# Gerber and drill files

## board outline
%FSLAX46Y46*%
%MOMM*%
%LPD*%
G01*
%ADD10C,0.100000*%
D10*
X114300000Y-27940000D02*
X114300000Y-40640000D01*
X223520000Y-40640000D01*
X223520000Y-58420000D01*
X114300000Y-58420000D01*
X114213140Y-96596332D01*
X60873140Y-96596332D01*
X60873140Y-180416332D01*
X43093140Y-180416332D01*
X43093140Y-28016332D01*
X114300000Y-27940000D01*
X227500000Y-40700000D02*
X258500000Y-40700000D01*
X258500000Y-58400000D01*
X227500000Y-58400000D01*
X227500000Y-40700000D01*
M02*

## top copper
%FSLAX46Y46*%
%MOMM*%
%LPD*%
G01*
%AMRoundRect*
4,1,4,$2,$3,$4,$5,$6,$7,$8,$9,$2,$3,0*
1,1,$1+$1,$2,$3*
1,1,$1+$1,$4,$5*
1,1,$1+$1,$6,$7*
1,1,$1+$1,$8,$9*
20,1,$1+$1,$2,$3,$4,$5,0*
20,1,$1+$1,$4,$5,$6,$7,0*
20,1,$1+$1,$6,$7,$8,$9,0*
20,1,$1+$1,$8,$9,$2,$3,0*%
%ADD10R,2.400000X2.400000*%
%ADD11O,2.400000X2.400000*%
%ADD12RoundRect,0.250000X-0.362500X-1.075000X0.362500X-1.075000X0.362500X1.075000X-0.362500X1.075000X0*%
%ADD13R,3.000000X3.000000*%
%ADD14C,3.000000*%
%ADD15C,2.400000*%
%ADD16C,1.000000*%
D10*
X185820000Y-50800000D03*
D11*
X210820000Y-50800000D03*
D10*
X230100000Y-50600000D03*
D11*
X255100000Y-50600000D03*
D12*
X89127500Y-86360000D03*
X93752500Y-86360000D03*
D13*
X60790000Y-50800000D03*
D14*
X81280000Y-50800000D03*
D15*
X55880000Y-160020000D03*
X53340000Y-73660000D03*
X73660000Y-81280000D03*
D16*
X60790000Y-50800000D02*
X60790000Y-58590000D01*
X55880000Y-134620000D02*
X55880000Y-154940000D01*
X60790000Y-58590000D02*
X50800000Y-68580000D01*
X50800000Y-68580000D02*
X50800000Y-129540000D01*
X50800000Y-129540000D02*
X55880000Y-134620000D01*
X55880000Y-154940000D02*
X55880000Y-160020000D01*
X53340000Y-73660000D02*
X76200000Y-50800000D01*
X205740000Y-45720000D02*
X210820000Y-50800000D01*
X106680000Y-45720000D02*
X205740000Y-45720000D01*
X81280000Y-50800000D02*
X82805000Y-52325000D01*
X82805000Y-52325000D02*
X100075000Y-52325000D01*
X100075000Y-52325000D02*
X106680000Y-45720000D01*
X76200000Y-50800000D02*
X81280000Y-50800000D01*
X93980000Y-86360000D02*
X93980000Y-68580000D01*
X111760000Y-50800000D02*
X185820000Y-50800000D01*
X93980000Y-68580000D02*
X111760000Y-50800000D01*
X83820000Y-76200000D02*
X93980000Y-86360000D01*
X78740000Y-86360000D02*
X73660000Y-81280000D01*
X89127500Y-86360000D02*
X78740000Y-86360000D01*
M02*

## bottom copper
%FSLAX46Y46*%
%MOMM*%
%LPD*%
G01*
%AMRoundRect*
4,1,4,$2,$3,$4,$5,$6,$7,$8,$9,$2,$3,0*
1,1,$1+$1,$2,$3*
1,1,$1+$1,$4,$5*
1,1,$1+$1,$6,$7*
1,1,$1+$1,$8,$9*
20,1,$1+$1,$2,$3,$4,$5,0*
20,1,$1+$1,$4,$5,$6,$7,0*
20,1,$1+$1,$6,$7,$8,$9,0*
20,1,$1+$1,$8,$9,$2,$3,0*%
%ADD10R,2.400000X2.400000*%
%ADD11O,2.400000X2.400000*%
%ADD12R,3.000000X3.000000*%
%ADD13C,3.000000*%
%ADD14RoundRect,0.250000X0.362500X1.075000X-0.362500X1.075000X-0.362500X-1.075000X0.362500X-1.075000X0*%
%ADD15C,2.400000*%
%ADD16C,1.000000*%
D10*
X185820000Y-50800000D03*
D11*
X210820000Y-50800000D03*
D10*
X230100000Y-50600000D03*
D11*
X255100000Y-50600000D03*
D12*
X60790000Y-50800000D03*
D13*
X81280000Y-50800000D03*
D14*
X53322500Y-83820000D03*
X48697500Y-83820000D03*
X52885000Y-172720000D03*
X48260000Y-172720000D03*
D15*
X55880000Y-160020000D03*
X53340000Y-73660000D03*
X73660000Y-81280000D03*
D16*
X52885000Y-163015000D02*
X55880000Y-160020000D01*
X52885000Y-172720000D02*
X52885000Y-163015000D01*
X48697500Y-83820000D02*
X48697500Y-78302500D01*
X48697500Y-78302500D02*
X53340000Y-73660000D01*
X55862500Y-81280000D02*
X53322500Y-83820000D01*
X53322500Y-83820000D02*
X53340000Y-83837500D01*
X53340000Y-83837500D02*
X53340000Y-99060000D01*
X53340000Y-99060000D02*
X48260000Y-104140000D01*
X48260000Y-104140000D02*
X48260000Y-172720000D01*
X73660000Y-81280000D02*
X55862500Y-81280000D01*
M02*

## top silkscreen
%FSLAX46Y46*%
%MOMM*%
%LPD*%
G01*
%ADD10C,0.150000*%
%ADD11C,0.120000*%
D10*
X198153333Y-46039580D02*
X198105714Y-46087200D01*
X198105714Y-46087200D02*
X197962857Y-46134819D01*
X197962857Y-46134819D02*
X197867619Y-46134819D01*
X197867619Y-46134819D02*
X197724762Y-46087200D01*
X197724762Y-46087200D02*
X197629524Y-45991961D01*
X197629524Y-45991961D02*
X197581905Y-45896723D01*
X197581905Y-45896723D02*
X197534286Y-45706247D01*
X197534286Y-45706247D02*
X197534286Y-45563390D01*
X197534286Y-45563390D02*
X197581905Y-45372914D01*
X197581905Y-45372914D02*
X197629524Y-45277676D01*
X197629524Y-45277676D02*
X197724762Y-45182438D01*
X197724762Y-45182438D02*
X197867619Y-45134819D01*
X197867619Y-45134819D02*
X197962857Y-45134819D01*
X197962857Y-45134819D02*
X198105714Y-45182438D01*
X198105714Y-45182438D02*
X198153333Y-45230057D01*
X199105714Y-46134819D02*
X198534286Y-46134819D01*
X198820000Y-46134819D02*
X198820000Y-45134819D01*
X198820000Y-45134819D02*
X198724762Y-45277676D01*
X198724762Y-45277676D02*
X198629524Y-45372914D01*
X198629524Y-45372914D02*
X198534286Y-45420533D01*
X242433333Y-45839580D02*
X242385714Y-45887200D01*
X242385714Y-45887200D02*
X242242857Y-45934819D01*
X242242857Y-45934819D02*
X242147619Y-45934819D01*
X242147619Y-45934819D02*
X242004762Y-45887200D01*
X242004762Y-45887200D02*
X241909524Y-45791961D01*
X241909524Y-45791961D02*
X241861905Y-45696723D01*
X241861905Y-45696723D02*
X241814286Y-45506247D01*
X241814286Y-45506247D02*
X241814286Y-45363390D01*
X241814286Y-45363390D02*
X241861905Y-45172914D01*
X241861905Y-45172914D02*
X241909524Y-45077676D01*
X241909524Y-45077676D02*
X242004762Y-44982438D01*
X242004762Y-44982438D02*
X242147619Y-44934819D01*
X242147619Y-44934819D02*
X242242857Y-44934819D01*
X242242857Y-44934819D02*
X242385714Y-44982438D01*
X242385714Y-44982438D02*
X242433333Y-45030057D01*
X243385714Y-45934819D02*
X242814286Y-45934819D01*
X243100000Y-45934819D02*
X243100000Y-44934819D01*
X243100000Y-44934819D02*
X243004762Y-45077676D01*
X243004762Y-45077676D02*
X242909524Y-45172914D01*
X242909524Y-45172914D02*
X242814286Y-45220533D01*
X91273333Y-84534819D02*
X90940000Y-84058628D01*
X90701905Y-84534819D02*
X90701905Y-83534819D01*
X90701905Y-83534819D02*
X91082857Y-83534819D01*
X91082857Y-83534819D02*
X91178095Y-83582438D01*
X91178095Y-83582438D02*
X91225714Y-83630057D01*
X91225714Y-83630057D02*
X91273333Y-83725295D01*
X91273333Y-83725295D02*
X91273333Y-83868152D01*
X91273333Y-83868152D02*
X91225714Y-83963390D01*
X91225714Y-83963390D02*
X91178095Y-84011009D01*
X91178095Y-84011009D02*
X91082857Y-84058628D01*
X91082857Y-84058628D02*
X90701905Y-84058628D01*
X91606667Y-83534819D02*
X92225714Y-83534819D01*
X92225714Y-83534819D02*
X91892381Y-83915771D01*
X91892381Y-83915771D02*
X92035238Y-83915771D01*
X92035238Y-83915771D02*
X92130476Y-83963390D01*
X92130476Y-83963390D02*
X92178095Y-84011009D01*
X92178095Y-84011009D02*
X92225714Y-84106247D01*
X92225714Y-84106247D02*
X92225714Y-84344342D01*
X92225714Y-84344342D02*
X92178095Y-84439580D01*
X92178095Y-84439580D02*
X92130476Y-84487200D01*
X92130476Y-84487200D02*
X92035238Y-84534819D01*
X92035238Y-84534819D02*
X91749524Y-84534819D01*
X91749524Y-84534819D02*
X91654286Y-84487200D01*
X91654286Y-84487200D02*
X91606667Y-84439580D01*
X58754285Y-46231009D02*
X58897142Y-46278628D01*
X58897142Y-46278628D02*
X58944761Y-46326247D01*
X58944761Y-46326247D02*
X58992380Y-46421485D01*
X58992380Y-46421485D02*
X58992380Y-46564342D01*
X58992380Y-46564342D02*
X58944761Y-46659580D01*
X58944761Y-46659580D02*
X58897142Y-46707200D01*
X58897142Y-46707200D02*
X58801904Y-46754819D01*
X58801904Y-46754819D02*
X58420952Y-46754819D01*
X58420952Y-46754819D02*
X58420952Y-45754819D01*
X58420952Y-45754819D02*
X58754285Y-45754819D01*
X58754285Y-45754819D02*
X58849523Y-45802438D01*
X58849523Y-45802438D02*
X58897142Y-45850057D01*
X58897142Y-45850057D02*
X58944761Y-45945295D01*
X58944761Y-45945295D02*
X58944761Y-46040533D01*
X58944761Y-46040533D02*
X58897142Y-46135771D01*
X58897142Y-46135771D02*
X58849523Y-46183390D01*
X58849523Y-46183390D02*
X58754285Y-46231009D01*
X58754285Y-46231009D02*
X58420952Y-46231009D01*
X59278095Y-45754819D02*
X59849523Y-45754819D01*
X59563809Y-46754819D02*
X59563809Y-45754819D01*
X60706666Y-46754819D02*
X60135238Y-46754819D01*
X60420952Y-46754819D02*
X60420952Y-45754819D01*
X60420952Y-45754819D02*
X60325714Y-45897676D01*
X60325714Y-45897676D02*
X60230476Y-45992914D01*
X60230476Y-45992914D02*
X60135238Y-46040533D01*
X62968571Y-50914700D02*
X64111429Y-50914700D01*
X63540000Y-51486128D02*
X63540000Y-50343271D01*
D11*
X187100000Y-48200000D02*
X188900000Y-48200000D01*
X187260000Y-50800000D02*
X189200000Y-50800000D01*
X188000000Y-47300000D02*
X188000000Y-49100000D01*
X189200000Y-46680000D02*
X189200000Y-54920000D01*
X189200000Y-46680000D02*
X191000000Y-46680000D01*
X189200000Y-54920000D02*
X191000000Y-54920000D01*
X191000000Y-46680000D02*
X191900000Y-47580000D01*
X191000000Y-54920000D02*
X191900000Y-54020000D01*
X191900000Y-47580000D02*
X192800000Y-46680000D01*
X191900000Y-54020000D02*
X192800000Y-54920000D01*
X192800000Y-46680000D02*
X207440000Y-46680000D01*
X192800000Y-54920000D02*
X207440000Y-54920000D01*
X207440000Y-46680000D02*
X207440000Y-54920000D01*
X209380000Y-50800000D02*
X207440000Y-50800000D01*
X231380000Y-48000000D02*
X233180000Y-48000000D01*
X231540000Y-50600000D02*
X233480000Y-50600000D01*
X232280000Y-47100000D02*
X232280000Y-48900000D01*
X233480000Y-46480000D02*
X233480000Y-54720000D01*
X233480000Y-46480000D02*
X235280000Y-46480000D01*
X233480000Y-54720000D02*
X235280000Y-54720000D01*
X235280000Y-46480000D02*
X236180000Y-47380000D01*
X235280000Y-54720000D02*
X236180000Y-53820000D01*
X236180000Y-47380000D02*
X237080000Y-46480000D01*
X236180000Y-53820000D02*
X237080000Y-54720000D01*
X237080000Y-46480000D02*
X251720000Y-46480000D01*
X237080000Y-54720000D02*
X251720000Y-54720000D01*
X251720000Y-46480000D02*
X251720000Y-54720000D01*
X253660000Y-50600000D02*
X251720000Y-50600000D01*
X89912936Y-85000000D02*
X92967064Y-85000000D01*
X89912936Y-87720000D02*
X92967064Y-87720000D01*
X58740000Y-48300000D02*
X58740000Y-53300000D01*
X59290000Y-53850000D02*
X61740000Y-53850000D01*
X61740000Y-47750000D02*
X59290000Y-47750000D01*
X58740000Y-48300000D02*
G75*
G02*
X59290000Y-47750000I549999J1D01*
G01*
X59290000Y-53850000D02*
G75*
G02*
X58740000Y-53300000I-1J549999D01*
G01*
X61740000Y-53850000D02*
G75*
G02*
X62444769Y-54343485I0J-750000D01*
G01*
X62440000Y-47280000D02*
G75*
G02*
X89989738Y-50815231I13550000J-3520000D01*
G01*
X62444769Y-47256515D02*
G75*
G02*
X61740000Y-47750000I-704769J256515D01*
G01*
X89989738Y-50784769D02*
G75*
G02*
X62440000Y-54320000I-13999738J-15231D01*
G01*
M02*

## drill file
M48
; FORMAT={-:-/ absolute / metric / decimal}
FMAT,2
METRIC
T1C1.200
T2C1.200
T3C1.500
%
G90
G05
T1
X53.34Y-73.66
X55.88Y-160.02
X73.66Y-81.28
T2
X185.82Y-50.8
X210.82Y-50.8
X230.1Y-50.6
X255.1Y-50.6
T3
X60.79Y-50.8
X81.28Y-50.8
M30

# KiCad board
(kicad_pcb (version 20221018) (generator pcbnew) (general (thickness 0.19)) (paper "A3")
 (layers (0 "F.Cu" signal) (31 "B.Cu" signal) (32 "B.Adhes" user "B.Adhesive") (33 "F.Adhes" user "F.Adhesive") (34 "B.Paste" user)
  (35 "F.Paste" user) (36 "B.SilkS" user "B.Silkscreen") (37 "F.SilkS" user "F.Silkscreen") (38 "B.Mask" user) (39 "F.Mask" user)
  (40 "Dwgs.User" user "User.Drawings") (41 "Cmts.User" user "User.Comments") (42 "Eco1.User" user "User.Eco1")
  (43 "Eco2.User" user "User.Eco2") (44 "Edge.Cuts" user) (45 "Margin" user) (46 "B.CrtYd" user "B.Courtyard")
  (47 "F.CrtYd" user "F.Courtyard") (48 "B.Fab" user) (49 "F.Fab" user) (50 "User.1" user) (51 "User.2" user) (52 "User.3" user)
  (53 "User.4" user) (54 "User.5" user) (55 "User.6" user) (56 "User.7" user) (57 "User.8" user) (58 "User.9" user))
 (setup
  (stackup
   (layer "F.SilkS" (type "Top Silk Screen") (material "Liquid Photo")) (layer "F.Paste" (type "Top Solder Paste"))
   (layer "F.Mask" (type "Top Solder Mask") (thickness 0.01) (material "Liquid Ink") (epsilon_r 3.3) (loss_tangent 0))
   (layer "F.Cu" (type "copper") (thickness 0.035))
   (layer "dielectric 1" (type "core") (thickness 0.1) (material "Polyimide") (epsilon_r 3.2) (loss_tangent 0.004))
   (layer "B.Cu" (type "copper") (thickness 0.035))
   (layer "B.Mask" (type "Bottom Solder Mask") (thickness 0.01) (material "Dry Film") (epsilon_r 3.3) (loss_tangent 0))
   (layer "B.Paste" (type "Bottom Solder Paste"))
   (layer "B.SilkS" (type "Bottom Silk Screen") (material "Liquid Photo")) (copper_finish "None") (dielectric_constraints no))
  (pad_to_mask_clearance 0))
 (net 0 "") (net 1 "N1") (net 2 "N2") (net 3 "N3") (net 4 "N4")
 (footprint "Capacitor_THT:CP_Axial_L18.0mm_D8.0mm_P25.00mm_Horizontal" (layer "F.Cu") (at 185.82 50.8)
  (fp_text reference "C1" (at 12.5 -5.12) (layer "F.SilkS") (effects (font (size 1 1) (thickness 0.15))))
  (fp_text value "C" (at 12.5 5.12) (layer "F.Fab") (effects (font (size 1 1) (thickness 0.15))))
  (fp_line (start 1.28 -2.6) (end 3.08 -2.6) (stroke (width 0.12) (type solid)) (layer "F.SilkS"))
  (fp_line (start 1.44 0) (end 3.38 0) (stroke (width 0.12) (type solid)) (layer "F.SilkS"))
  (fp_line (start 2.18 -3.5) (end 2.18 -1.7) (stroke (width 0.12) (type solid)) (layer "F.SilkS"))
  (fp_line (start 3.38 -4.12) (end 3.38 4.12) (stroke (width 0.12) (type solid)) (layer "F.SilkS"))
  (fp_line (start 3.38 -4.12) (end 5.18 -4.12) (stroke (width 0.12) (type solid)) (layer "F.SilkS"))
  (fp_line (start 3.38 4.12) (end 5.18 4.12) (stroke (width 0.12) (type solid)) (layer "F.SilkS"))
  (fp_line (start 5.18 -4.12) (end 6.08 -3.22) (stroke (width 0.12) (type solid)) (layer "F.SilkS"))
  (fp_line (start 5.18 4.12) (end 6.08 3.22) (stroke (width 0.12) (type solid)) (layer "F.SilkS"))
  (fp_line (start 6.08 -3.22) (end 6.98 -4.12) (stroke (width 0.12) (type solid)) (layer "F.SilkS"))
  (fp_line (start 6.08 3.22) (end 6.98 4.12) (stroke (width 0.12) (type solid)) (layer "F.SilkS"))
  (fp_line (start 6.98 -4.12) (end 21.62 -4.12) (stroke (width 0.12) (type solid)) (layer "F.SilkS"))
  (fp_line (start 6.98 4.12) (end 21.62 4.12) (stroke (width 0.12) (type solid)) (layer "F.SilkS"))
  (fp_line (start 21.62 -4.12) (end 21.62 4.12) (stroke (width 0.12) (type solid)) (layer "F.SilkS"))
  (fp_line (start 23.56 0) (end 21.62 0) (stroke (width 0.12) (type solid)) (layer "F.SilkS"))
  (pad "1" thru_hole rect (at 0 0) (size 2.4 2.4) (drill 1.2) (layers "*.Cu" "*.Mask") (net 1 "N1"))
  (pad "2" thru_hole oval (at 25 0) (size 2.4 2.4) (drill 1.2) (layers "*.Cu" "*.Mask") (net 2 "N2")))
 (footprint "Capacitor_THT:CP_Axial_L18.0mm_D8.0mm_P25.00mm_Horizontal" (layer "F.Cu") (at 230.1 50.6)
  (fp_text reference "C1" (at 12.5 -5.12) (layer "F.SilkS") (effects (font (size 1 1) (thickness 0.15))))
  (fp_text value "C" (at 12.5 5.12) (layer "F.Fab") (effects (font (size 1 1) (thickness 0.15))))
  (fp_line (start 1.28 -2.6) (end 3.08 -2.6) (stroke (width 0.12) (type solid)) (layer "F.SilkS"))
  (fp_line (start 1.44 0) (end 3.38 0) (stroke (width 0.12) (type solid)) (layer "F.SilkS"))
  (fp_line (start 2.18 -3.5) (end 2.18 -1.7) (stroke (width 0.12) (type solid)) (layer "F.SilkS"))
  (fp_line (start 3.38 -4.12) (end 3.38 4.12) (stroke (width 0.12) (type solid)) (layer "F.SilkS"))
  (fp_line (start 3.38 -4.12) (end 5.18 -4.12) (stroke (width 0.12) (type solid)) (layer "F.SilkS"))
  (fp_line (start 3.38 4.12) (end 5.18 4.12) (stroke (width 0.12) (type solid)) (layer "F.SilkS"))
  (fp_line (start 5.18 -4.12) (end 6.08 -3.22) (stroke (width 0.12) (type solid)) (layer "F.SilkS"))
  (fp_line (start 5.18 4.12) (end 6.08 3.22) (stroke (width 0.12) (type solid)) (layer "F.SilkS"))
  (fp_line (start 6.08 -3.22) (end 6.98 -4.12) (stroke (width 0.12) (type solid)) (layer "F.SilkS"))
  (fp_line (start 6.08 3.22) (end 6.98 4.12) (stroke (width 0.12) (type solid)) (layer "F.SilkS"))
  (fp_line (start 6.98 -4.12) (end 21.62 -4.12) (stroke (width 0.12) (type solid)) (layer "F.SilkS"))
  (fp_line (start 6.98 4.12) (end 21.62 4.12) (stroke (width 0.12) (type solid)) (layer "F.SilkS"))
  (fp_line (start 21.62 -4.12) (end 21.62 4.12) (stroke (width 0.12) (type solid)) (layer "F.SilkS"))
  (fp_line (start 23.56 0) (end 21.62 0) (stroke (width 0.12) (type solid)) (layer "F.SilkS"))
  (pad "1" thru_hole rect (at 0 0) (size 2.4 2.4) (drill 1.2) (layers "*.Cu" "*.Mask"))
  (pad "2" thru_hole oval (at 25 0) (size 2.4 2.4) (drill 1.2) (layers "*.Cu" "*.Mask")))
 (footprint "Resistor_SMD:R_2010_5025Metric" (layer "F.Cu") (at 91.44 86.36)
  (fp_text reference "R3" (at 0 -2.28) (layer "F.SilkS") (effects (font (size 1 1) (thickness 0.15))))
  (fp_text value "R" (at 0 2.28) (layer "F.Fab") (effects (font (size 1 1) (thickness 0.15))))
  (fp_line (start -1.527064 -1.36) (end 1.527064 -1.36) (stroke (width 0.12) (type solid)) (layer "F.SilkS"))
  (fp_line (start -1.527064 1.36) (end 1.527064 1.36) (stroke (width 0.12) (type solid)) (layer "F.SilkS"))
  (pad "1" smd roundrect (at -2.3125 0) (size 1.225 2.65) (layers "F.Cu" "F.Paste" "F.Mask") (roundrect_rratio 0.204082) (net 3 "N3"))
  (pad "2" smd roundrect (at 2.3125 0) (size 1.225 2.65) (layers "F.Cu" "F.Paste" "F.Mask") (roundrect_rratio 0.204082) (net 1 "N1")))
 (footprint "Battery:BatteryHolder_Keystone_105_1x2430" (layer "F.Cu") (at 60.79 50.8)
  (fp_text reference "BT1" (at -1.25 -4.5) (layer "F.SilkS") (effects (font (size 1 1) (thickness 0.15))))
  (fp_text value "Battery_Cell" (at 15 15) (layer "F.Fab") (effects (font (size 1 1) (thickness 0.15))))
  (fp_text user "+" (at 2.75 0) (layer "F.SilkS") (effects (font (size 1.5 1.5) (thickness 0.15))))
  (fp_line (start -2.05 -2.5) (end -2.05 2.5) (stroke (width 0.12) (type solid)) (layer "F.SilkS"))
  (fp_line (start -1.5 3.05) (end 0.95 3.05) (stroke (width 0.12) (type solid)) (layer "F.SilkS"))
  (fp_line (start 0.95 -3.05) (end -1.5 -3.05) (stroke (width 0.12) (type solid)) (layer "F.SilkS"))
  (fp_arc (start -2.05 -2.5) (mid -1.888909 -2.888909) (end -1.5 -3.05) (stroke (width 0.12) (type solid)) (layer "F.SilkS"))
  (fp_arc (start -1.5 3.05) (mid -1.888909 2.888909) (end -2.05 2.5) (stroke (width 0.12) (type solid)) (layer "F.SilkS"))
  (fp_arc (start 0.95 3.05) (mid 1.380182 3.185636) (end 1.654769 3.543485) (stroke (width 0.12) (type solid)) (layer "F.SilkS"))
  (fp_arc (start 1.65 -3.52) (mid 16.981862 -13.885887) (end 29.199738 0.015231) (stroke (width 0.12) (type solid)) (layer "F.SilkS"))
  (fp_arc (start 1.654769 -3.543485) (mid 1.380182 -3.185636) (end 0.95 -3.05) (stroke (width 0.12) (type solid)) (layer "F.SilkS"))
  (fp_arc (start 29.199738 -0.015231) (mid 16.981862 13.885887) (end 1.65 3.52) (stroke (width 0.12) (type solid)) (layer "F.SilkS"))
  (pad "1" thru_hole rect (at 0 0) (size 3 3) (drill 1.5) (layers "*.Cu" "*.Mask") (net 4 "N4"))
  (pad "2" thru_hole circle (at 20.49 0) (size 3 3) (drill 1.5) (layers "*.Cu" "*.Mask") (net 2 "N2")))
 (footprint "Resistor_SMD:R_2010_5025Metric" (layer "B.Cu") (at 51.01 83.82 180)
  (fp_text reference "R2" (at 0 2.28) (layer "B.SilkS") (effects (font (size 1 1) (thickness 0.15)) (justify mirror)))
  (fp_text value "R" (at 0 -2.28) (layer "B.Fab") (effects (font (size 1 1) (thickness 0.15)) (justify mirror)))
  (pad "1" smd roundrect (at -2.3125 0 180) (size 1.225 2.65) (layers "B.Cu" "B.Paste" "B.Mask") (roundrect_rratio 0.204082) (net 3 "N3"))
  (pad "2" smd roundrect (at 2.3125 0 180) (size 1.225 2.65) (layers "B.Cu" "B.Paste" "B.Mask") (roundrect_rratio 0.204082) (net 2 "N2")))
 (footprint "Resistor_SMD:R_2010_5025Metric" (layer "B.Cu") (at 50.5725 172.72 180)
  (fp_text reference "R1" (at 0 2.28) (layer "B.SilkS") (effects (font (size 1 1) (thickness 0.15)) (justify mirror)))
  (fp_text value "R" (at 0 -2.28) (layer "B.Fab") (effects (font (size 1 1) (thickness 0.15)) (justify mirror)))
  (pad "1" smd roundrect (at -2.3125 0 180) (size 1.225 2.65) (layers "B.Cu" "B.Paste" "B.Mask") (roundrect_rratio 0.204082) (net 4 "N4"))
  (pad "2" smd roundrect (at 2.3125 0 180) (size 1.225 2.65) (layers "B.Cu" "B.Paste" "B.Mask") (roundrect_rratio 0.204082) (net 3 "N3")))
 (gr_poly
  (pts (xy 114.3 27.94) (xy 114.3 40.64) (xy 223.52 40.64) (xy 223.52 58.42) (xy 114.3 58.42) (xy 114.21314 96.596332)
   (xy 60.87314 96.596332) (xy 60.87314 180.416332) (xy 43.09314 180.416332) (xy 43.09314 28.016332))
  (stroke (width 0.1) (type solid)) (fill none) (layer "Edge.Cuts"))
 (gr_rect (start 227.5 40.7) (end 258.5 58.4) (stroke (width 0.1) (type default)) (fill none) (layer "Edge.Cuts"))
 (segment (start 60.79 50.8) (end 60.79 58.59) (width 1) (layer "F.Cu") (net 4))
 (segment (start 55.88 134.62) (end 55.88 154.94) (width 1) (layer "F.Cu") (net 4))
 (segment (start 60.79 58.59) (end 50.8 68.58) (width 1) (layer "F.Cu") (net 4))
 (segment (start 50.8 68.58) (end 50.8 129.54) (width 1) (layer "F.Cu") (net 4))
 (segment (start 50.8 129.54) (end 55.88 134.62) (width 1) (layer "F.Cu") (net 4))
 (segment (start 55.88 154.94) (end 55.88 160.02) (width 1) (layer "F.Cu") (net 4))
 (via (at 55.88 160.02) (size 2.4) (drill 1.2) (layers "F.Cu" "B.Cu") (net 4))
 (segment (start 52.885 163.015) (end 55.88 160.02) (width 1) (layer "B.Cu") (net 4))
 (segment (start 52.885 172.72) (end 52.885 163.015) (width 1) (layer "B.Cu") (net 4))
 (segment (start 53.34 73.66) (end 76.2 50.8) (width 1) (layer "F.Cu") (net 2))
 (segment (start 205.74 45.72) (end 210.82 50.8) (width 1) (layer "F.Cu") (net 2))
 (segment (start 106.68 45.72) (end 205.74 45.72) (width 1) (layer "F.Cu") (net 2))
 (segment (start 81.28 50.8) (end 82.805 52.325) (width 1) (layer "F.Cu") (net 2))
 (segment (start 82.805 52.325) (end 100.075 52.325) (width 1) (layer "F.Cu") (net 2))
 (segment (start 100.075 52.325) (end 106.68 45.72) (width 1) (layer "F.Cu") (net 2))
 (segment (start 76.2 50.8) (end 81.28 50.8) (width 1) (layer "F.Cu") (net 2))
 (via (at 53.34 73.66) (size 2.4) (drill 1.2) (layers "F.Cu" "B.Cu") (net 2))
 (segment (start 48.6975 83.82) (end 48.6975 78.3025) (width 1) (layer "B.Cu") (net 2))
 (segment (start 48.6975 78.3025) (end 53.34 73.66) (width 1) (layer "B.Cu") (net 2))
 (segment (start 93.98 86.36) (end 93.98 68.58) (width 1) (layer "F.Cu") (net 1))
 (segment (start 111.76 50.8) (end 185.82 50.8) (width 1) (layer "F.Cu") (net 1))
 (segment (start 93.98 68.58) (end 111.76 50.8) (width 1) (layer "F.Cu") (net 1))
 (segment (start 83.82 76.2) (end 93.98 86.36) (width 1) (layer "F.Cu") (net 1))
 (segment (start 78.74 86.36) (end 73.66 81.28) (width 1) (layer "F.Cu") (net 3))
 (segment (start 89.1275 86.36) (end 78.74 86.36) (width 1) (layer "F.Cu") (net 3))
 (via (at 73.66 81.28) (size 2.4) (drill 1.2) (layers "F.Cu" "B.Cu") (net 3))
 (segment (start 55.8625 81.28) (end 53.3225 83.82) (width 1) (layer "B.Cu") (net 3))
 (segment (start 53.3225 83.82) (end 53.34 83.8375) (width 1) (layer "B.Cu") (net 3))
 (segment (start 53.34 83.8375) (end 53.34 99.06) (width 1) (layer "B.Cu") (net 3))
 (segment (start 53.34 99.06) (end 48.26 104.14) (width 1) (layer "B.Cu") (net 3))
 (segment (start 48.26 104.14) (end 48.26 172.72) (width 1) (layer "B.Cu") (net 3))
 (segment (start 73.66 81.28) (end 55.8625 81.28) (width 1) (layer "B.Cu") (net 3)))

